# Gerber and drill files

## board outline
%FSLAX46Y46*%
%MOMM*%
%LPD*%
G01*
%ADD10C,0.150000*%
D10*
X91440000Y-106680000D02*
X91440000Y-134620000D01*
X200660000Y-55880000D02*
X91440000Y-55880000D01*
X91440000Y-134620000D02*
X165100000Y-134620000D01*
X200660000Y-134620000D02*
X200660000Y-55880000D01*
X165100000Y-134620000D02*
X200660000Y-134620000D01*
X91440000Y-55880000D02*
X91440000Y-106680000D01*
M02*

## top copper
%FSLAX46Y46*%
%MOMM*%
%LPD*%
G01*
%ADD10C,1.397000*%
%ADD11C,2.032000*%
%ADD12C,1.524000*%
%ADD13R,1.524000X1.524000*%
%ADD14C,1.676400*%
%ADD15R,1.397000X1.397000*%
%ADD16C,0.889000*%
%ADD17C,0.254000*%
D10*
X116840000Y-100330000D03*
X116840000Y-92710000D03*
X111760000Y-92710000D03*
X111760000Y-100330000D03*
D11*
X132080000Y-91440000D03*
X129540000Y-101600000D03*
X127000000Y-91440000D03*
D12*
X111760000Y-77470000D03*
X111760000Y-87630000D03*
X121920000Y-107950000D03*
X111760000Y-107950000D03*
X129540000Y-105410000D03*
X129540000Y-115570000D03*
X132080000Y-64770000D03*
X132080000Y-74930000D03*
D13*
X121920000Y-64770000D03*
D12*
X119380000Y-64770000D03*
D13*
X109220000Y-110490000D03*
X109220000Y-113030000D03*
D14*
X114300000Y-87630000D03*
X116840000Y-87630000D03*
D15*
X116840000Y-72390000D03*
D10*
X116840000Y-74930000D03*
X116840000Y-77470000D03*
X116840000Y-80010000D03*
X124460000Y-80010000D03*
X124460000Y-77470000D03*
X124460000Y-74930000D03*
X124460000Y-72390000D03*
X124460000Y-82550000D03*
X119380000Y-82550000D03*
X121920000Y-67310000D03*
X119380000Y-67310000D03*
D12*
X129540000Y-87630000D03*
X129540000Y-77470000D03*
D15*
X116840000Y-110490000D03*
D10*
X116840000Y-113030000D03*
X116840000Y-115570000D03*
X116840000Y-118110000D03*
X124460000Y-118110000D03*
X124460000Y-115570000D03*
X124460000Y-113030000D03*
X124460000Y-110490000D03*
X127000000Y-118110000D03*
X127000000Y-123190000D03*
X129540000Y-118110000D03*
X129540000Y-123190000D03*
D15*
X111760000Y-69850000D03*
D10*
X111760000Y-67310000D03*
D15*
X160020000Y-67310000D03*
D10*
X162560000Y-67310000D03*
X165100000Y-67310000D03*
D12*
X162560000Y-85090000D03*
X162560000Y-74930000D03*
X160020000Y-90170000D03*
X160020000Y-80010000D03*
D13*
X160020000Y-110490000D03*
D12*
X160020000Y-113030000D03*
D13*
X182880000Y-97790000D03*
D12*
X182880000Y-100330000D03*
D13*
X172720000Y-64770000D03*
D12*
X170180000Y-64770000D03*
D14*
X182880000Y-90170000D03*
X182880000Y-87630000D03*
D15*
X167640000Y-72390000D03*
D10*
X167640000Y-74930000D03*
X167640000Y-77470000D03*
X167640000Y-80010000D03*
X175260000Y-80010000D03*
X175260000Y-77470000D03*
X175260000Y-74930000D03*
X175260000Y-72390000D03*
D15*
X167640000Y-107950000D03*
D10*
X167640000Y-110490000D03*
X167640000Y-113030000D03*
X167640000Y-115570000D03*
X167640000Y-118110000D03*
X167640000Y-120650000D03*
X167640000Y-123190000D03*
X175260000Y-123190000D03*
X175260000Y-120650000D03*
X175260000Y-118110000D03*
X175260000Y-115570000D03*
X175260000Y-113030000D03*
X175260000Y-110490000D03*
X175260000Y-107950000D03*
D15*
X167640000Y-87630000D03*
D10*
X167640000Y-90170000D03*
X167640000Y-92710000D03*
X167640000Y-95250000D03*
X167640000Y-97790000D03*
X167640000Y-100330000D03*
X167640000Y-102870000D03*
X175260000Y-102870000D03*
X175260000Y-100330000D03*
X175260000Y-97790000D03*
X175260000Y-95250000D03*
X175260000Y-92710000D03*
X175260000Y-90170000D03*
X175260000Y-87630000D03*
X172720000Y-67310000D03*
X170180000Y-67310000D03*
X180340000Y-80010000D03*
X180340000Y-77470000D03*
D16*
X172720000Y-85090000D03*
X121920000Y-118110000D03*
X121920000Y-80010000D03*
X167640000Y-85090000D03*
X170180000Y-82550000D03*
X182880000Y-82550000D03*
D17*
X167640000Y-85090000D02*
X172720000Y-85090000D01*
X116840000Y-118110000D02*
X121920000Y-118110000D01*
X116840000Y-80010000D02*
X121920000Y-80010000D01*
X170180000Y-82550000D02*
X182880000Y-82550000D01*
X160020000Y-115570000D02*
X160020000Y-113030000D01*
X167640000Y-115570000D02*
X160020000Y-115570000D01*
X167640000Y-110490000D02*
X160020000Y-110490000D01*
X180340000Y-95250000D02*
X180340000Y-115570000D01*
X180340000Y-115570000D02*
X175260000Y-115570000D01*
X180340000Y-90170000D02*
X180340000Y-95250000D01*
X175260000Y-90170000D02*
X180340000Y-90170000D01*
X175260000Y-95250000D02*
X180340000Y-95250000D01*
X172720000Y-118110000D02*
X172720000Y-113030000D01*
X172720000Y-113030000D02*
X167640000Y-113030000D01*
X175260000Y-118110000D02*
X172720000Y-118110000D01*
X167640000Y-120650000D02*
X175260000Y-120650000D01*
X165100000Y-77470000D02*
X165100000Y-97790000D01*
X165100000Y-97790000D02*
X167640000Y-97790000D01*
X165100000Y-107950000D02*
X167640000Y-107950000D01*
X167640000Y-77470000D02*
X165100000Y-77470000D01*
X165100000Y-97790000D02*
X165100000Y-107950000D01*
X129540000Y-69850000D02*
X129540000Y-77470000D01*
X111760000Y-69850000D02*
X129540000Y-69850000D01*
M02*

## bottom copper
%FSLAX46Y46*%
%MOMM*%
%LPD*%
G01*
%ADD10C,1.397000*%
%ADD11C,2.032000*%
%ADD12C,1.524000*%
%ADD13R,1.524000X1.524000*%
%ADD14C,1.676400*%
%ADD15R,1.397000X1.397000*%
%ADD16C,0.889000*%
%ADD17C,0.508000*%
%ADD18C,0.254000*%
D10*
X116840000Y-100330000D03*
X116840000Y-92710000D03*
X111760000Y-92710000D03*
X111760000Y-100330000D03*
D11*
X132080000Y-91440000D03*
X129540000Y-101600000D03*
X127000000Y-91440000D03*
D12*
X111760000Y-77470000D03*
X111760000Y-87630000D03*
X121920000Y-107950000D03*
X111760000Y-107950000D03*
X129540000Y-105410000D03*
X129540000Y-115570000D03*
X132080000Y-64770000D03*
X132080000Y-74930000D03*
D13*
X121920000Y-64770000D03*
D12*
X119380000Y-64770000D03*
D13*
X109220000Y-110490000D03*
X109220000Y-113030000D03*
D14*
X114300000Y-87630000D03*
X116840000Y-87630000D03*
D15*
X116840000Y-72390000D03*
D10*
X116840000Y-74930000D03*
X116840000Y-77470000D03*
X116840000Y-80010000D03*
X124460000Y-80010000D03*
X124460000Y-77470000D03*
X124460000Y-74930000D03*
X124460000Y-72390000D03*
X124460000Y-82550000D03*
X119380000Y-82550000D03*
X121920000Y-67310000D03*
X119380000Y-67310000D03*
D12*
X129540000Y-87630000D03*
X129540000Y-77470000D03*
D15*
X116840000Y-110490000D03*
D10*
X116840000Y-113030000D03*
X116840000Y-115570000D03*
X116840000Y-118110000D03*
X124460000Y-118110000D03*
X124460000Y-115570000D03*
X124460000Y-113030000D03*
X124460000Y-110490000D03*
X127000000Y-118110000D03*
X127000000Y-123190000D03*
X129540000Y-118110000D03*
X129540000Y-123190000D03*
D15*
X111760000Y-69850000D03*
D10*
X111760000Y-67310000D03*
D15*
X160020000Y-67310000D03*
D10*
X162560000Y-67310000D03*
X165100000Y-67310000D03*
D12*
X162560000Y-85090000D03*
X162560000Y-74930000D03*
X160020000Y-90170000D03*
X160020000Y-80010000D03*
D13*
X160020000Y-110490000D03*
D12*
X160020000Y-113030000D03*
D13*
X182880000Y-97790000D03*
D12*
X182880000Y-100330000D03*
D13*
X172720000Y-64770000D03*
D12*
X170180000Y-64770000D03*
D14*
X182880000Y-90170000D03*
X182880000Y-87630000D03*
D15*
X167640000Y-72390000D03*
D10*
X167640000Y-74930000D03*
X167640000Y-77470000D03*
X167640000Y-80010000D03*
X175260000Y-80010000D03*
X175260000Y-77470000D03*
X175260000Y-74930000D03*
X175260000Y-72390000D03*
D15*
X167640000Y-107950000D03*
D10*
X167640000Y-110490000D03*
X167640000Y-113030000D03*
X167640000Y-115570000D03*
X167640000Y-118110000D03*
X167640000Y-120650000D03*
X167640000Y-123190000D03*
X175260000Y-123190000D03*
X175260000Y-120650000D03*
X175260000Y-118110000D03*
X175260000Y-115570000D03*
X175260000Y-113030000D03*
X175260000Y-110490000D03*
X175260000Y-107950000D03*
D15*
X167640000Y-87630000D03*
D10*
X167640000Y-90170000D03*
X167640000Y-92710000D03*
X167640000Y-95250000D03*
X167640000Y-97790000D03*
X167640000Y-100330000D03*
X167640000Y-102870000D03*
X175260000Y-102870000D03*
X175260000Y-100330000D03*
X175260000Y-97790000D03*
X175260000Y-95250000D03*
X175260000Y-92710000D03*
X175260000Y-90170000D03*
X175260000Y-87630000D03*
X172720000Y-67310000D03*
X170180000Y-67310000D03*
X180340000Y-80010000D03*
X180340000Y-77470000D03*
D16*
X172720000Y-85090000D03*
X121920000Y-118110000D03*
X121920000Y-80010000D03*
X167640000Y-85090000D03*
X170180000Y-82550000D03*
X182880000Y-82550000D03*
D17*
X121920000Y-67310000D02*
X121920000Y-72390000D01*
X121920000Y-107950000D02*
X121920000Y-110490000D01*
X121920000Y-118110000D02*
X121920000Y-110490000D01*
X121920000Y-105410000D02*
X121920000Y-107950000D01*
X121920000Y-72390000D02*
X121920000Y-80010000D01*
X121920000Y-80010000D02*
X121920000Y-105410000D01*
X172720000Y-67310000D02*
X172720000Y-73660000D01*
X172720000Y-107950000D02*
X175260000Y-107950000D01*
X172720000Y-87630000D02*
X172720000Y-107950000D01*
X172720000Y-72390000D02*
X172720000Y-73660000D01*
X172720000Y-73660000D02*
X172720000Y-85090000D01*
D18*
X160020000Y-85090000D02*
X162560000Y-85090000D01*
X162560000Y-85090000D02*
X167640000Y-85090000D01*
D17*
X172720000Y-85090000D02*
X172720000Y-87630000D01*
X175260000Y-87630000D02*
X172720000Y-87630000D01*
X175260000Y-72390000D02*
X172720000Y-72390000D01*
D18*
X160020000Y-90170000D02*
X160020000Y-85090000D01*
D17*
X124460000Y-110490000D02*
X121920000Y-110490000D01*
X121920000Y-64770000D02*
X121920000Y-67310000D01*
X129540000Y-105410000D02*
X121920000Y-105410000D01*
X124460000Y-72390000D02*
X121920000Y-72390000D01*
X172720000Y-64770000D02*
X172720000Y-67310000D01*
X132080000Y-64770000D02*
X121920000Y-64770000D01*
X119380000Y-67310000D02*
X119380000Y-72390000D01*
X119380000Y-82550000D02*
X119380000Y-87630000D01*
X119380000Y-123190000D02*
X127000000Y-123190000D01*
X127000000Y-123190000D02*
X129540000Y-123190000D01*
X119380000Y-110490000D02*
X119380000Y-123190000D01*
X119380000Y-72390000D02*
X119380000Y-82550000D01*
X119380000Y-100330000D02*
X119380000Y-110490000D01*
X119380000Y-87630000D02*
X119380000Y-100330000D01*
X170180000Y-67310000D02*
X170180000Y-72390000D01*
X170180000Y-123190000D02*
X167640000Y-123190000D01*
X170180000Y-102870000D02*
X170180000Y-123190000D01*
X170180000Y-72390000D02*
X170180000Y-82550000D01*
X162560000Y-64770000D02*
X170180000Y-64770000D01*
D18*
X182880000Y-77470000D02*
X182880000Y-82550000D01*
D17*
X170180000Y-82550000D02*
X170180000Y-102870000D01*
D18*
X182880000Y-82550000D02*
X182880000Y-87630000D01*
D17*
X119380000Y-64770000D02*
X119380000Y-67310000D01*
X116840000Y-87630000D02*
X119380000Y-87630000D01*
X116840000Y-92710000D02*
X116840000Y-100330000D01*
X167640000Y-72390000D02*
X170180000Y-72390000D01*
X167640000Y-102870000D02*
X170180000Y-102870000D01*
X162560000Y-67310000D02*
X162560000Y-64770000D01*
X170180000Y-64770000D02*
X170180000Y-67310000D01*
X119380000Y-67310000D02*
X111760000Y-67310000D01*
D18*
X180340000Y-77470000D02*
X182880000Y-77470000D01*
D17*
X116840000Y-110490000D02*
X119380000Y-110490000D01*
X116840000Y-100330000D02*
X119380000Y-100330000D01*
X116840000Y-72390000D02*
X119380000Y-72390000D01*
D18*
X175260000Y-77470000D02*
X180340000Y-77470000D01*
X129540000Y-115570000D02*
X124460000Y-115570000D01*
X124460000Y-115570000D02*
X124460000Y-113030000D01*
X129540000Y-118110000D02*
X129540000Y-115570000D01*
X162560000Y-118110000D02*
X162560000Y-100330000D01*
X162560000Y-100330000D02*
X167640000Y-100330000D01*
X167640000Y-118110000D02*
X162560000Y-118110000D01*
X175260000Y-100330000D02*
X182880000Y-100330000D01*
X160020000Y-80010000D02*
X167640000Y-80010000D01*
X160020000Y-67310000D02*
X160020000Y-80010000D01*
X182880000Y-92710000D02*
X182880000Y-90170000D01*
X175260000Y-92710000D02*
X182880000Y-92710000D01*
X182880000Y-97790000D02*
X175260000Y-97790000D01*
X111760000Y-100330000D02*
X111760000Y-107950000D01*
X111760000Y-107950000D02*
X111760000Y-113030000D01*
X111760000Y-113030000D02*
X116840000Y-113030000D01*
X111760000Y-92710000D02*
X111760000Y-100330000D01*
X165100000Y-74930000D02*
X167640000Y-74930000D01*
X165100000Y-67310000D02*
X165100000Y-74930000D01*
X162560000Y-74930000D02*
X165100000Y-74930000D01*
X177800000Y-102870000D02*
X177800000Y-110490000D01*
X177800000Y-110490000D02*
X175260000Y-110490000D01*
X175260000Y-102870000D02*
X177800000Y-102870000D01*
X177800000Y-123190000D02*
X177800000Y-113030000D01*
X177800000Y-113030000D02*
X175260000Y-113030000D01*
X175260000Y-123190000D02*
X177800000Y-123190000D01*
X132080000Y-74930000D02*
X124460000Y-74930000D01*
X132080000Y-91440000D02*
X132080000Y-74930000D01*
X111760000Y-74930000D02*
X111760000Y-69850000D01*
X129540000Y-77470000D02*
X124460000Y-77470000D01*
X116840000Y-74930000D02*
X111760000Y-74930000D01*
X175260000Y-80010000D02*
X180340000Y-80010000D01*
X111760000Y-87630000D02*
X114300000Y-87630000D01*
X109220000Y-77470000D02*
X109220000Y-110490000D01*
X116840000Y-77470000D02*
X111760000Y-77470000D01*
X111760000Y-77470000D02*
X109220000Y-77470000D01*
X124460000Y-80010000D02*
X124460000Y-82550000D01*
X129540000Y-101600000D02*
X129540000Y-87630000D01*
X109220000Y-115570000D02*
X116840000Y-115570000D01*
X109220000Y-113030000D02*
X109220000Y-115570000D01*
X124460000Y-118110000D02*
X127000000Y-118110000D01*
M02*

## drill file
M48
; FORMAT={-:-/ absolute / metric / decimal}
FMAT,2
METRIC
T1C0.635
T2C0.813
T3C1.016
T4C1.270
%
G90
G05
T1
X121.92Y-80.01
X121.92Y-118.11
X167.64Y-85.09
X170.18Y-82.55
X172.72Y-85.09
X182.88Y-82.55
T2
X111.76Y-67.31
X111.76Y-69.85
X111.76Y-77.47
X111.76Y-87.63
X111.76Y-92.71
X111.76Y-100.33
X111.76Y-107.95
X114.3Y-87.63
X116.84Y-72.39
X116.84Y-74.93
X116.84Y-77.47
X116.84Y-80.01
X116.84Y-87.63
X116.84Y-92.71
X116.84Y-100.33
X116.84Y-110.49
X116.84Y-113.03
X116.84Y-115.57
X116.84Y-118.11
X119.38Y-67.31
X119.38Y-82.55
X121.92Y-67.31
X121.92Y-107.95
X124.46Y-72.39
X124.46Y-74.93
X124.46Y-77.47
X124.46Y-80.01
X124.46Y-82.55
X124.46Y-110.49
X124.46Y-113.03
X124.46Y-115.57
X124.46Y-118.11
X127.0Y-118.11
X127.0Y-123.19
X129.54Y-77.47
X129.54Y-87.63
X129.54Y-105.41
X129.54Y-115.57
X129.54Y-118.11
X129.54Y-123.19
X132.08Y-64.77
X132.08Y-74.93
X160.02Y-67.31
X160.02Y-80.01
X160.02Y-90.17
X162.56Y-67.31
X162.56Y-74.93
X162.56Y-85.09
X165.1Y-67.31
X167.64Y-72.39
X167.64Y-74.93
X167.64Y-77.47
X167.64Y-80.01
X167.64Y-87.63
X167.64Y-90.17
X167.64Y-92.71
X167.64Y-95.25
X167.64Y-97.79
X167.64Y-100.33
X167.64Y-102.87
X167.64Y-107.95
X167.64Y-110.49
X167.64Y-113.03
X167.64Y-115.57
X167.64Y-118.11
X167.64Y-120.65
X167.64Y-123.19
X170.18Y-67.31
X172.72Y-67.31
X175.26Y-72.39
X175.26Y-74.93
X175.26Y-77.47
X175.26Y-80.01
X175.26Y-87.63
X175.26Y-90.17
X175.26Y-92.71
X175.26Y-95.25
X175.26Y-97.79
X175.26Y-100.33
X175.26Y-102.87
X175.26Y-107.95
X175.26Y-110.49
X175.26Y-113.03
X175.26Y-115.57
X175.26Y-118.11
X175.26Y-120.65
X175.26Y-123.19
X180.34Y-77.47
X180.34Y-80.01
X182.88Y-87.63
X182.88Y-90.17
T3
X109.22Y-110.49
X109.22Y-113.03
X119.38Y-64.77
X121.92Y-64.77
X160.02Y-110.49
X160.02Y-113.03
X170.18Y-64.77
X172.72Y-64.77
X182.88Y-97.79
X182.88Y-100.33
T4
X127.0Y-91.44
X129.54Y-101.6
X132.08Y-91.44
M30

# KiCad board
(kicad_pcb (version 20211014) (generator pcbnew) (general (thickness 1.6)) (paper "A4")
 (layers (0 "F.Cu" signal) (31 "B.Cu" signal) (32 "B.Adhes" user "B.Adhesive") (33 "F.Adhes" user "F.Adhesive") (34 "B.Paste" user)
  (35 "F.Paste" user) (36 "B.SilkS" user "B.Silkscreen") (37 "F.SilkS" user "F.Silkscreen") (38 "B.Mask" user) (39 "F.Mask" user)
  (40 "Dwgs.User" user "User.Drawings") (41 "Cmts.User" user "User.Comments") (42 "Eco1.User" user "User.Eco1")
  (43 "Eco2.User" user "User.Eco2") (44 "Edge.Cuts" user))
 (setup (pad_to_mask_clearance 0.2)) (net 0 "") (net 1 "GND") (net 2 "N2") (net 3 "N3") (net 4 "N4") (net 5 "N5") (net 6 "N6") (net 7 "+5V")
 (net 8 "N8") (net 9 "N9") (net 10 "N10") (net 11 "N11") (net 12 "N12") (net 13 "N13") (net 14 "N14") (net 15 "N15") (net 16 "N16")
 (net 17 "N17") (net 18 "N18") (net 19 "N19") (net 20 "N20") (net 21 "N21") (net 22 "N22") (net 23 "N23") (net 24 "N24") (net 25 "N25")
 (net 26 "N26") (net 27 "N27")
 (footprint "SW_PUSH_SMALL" (layer "F.Cu") (at 114.3 96.52 -90)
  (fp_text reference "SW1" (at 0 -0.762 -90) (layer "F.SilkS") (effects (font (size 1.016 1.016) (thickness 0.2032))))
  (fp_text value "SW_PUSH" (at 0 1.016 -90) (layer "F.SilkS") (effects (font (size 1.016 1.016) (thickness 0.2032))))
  (pad "1" thru_hole circle locked (at 3.81 -2.54 270) (size 1.397 1.397) (drill 0.8128) (layers *.Cu *.Mask "F.SilkS") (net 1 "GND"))
  (pad "1" thru_hole circle locked (at -3.81 -2.54 270) (size 1.397 1.397) (drill 0.8128) (layers *.Cu *.Mask "F.SilkS") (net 1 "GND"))
  (pad "2" thru_hole circle locked (at -3.81 2.54 270) (size 1.397 1.397) (drill 0.8128) (layers *.Cu *.Mask "F.SilkS") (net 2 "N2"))
  (pad "2" thru_hole circle locked (at 3.81 2.54 270) (size 1.397 1.397) (drill 0.8128) (layers *.Cu *.Mask "F.SilkS") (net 2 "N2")))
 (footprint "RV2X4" (layer "F.Cu") (at 129.54 96.52 -90)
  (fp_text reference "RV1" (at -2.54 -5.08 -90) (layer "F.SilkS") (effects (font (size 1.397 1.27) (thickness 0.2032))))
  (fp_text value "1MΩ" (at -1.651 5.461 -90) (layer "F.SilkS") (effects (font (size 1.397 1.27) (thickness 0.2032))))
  (pad "1" thru_hole circle locked (at -5.08 -2.54 270) (size 2.032 2.032) (drill 1.27) (layers *.Cu *.Mask "F.SilkS") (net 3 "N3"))
  (pad "2" thru_hole circle locked (at 5.08 0 270) (size 2.032 2.032) (drill 1.27) (layers *.Cu *.Mask "F.SilkS") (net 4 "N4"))
  (pad "3" thru_hole circle locked (at -5.08 2.54 270) (size 2.032 2.032) (drill 1.27) (layers *.Cu *.Mask "F.SilkS")))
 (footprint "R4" (layer "F.Cu") (at 111.76 82.55 -90) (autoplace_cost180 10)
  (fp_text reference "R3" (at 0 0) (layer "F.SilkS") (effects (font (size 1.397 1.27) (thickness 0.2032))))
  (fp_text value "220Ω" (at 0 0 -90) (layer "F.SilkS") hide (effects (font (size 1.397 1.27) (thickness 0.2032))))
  (pad "1" thru_hole circle locked (at -5.08 0 270) (size 1.524 1.524) (drill 0.8128) (layers *.Cu *.Mask "F.SilkS") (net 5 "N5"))
  (pad "2" thru_hole circle locked (at 5.08 0 270) (size 1.524 1.524) (drill 0.8128) (layers *.Cu *.Mask "F.SilkS") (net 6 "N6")))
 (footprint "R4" (layer "F.Cu") (at 116.84 107.95 180) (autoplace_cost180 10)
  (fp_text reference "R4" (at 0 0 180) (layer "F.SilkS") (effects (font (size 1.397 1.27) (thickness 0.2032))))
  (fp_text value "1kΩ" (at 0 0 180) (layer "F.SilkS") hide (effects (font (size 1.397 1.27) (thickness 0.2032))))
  (pad "1" thru_hole circle locked (at -5.08 0 180) (size 1.524 1.524) (drill 0.8128) (layers *.Cu *.Mask "F.SilkS") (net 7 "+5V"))
  (pad "2" thru_hole circle locked (at 5.08 0 180) (size 1.524 1.524) (drill 0.8128) (layers *.Cu *.Mask "F.SilkS") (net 2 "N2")))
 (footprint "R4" (layer "F.Cu") (at 129.54 110.49 -90) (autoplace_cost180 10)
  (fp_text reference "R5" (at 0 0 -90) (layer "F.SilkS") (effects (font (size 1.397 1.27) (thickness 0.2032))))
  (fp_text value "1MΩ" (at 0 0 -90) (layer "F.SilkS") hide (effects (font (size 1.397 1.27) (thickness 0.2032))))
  (pad "1" thru_hole circle locked (at -5.08 0 270) (size 1.524 1.524) (drill 0.8128) (layers *.Cu *.Mask "F.SilkS") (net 7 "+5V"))
  (pad "2" thru_hole circle locked (at 5.08 0 270) (size 1.524 1.524) (drill 0.8128) (layers *.Cu *.Mask "F.SilkS") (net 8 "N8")))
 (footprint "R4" (layer "F.Cu") (at 132.08 69.85 -90) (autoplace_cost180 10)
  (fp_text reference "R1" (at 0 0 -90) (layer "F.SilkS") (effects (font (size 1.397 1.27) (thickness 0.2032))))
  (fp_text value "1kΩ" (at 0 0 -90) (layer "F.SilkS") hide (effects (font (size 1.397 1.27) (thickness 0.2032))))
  (pad "1" thru_hole circle locked (at -5.08 0 270) (size 1.524 1.524) (drill 0.8128) (layers *.Cu *.Mask "F.SilkS") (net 7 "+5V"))
  (pad "2" thru_hole circle locked (at 5.08 0 270) (size 1.524 1.524) (drill 0.8128) (layers *.Cu *.Mask "F.SilkS") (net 3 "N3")))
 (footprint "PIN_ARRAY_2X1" (layer "F.Cu") (at 120.65 64.77 180)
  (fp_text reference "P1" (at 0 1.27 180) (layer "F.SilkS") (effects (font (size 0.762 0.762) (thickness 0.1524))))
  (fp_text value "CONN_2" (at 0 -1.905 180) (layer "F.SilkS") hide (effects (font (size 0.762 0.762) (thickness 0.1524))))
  (pad "1" thru_hole rect locked (at -1.27 0 180) (size 1.524 1.524) (drill 1.016) (layers *.Cu *.Mask "F.SilkS") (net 7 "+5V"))
  (pad "2" thru_hole circle locked (at 1.27 0 180) (size 1.524 1.524) (drill 1.016) (layers *.Cu *.Mask "F.SilkS") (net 1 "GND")))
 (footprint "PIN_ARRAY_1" (layer "F.Cu") (at 109.22 110.49)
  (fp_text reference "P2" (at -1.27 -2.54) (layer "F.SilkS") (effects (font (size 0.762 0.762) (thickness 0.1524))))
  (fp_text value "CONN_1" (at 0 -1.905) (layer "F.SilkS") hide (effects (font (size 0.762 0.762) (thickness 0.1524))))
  (pad "1" thru_hole rect locked (at 0 0) (size 1.524 1.524) (drill 1.016) (layers *.Cu *.Mask "F.SilkS") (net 5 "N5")))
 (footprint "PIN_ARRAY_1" (layer "F.Cu") (at 109.22 113.03)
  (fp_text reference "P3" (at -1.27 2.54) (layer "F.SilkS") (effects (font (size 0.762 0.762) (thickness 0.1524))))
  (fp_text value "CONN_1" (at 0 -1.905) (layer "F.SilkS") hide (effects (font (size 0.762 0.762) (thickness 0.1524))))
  (pad "1" thru_hole rect locked (at 0 0) (size 1.524 1.524) (drill 1.016) (layers *.Cu *.Mask "F.SilkS") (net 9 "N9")))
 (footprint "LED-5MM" (layer "F.Cu") (at 115.57 87.63)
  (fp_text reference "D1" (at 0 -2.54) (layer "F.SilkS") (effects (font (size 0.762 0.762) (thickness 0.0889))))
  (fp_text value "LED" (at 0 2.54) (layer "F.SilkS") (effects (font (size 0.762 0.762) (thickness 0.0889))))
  (pad "1" thru_hole circle locked (at -1.27 0) (size 1.6764 1.6764) (drill 0.8128) (layers *.Cu *.Mask "F.SilkS") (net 6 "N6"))
  (pad "2" thru_hole circle locked (at 1.27 0) (size 1.6764 1.6764) (drill 0.8128) (layers *.Cu *.Mask "F.SilkS") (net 1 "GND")))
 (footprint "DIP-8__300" (layer "F.Cu") (at 120.65 76.2 -90)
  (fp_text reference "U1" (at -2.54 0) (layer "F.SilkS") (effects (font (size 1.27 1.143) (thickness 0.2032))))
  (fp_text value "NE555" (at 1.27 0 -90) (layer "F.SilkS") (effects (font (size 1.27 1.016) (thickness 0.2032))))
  (pad "1" thru_hole rect locked (at -3.81 3.81 270) (size 1.397 1.397) (drill 0.8128) (layers *.Cu *.Mask "F.SilkS") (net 1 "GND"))
  (pad "2" thru_hole circle locked (at -1.27 3.81 270) (size 1.397 1.397) (drill 0.8128) (layers *.Cu *.Mask "F.SilkS") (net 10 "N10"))
  (pad "3" thru_hole circle locked (at 1.27 3.81 270) (size 1.397 1.397) (drill 0.8128) (layers *.Cu *.Mask "F.SilkS") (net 5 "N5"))
  (pad "4" thru_hole circle locked (at 3.81 3.81 270) (size 1.397 1.397) (drill 0.8128) (layers *.Cu *.Mask "F.SilkS") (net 7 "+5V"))
  (pad "5" thru_hole circle locked (at 3.81 -3.81 270) (size 1.397 1.397) (drill 0.8128) (layers *.Cu *.Mask "F.SilkS") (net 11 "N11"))
  (pad "6" thru_hole circle locked (at 1.27 -3.81 270) (size 1.397 1.397) (drill 0.8128) (layers *.Cu *.Mask "F.SilkS") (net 10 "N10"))
  (pad "7" thru_hole circle locked (at -1.27 -3.81 270) (size 1.397 1.397) (drill 0.8128) (layers *.Cu *.Mask "F.SilkS") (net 3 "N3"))
  (pad "8" thru_hole circle locked (at -3.81 -3.81 270) (size 1.397 1.397) (drill 0.8128) (layers *.Cu *.Mask "F.SilkS") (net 7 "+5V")))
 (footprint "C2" (layer "F.Cu") (at 121.92 82.55 180)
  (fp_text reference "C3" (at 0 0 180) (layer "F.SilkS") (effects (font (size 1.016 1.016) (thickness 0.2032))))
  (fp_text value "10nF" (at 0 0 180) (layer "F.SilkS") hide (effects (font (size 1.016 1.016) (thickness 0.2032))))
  (pad "1" thru_hole circle locked (at -2.54 0 180) (size 1.397 1.397) (drill 0.8128) (layers *.Cu *.Mask "F.SilkS") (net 11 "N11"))
  (pad "2" thru_hole circle locked (at 2.54 0 180) (size 1.397 1.397) (drill 0.8128) (layers *.Cu *.Mask "F.SilkS") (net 1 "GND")))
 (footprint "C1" (layer "F.Cu") (at 120.65 67.31 180)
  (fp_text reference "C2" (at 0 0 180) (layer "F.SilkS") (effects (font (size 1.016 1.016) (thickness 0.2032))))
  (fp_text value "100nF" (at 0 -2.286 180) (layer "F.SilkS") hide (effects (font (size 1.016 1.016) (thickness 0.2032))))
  (pad "1" thru_hole circle locked (at -1.27 0 180) (size 1.397 1.397) (drill 0.8128) (layers *.Cu *.Mask "F.SilkS") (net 7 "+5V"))
  (pad "2" thru_hole circle locked (at 1.27 0 180) (size 1.397 1.397) (drill 0.8128) (layers *.Cu *.Mask "F.SilkS") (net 1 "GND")))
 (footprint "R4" (layer "F.Cu") (at 129.54 82.55 90) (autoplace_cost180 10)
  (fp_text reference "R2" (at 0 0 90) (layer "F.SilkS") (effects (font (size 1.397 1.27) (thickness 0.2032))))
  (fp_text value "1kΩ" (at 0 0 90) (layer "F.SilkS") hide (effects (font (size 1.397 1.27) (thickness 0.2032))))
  (pad "1" thru_hole circle locked (at -5.08 0 90) (size 1.524 1.524) (drill 0.8128) (layers *.Cu *.Mask "F.SilkS") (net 4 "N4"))
  (pad "2" thru_hole circle locked (at 5.08 0 90) (size 1.524 1.524) (drill 0.8128) (layers *.Cu *.Mask "F.SilkS") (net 10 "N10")))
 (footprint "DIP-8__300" (layer "F.Cu") (at 120.65 114.3 -90)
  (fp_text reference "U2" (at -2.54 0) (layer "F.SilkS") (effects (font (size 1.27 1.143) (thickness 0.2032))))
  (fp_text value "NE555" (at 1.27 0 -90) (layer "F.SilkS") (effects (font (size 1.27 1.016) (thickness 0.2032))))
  (pad "1" thru_hole rect locked (at -3.81 3.81 270) (size 1.397 1.397) (drill 0.8128) (layers *.Cu *.Mask "F.SilkS") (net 1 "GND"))
  (pad "2" thru_hole circle locked (at -1.27 3.81 270) (size 1.397 1.397) (drill 0.8128) (layers *.Cu *.Mask "F.SilkS") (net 2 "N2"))
  (pad "3" thru_hole circle locked (at 1.27 3.81 270) (size 1.397 1.397) (drill 0.8128) (layers *.Cu *.Mask "F.SilkS") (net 9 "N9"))
  (pad "4" thru_hole circle locked (at 3.81 3.81 270) (size 1.397 1.397) (drill 0.8128) (layers *.Cu *.Mask "F.SilkS") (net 7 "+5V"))
  (pad "5" thru_hole circle locked (at 3.81 -3.81 270) (size 1.397 1.397) (drill 0.8128) (layers *.Cu *.Mask "F.SilkS") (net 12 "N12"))
  (pad "6" thru_hole circle locked (at 1.27 -3.81 270) (size 1.397 1.397) (drill 0.8128) (layers *.Cu *.Mask "F.SilkS") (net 8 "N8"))
  (pad "7" thru_hole circle locked (at -1.27 -3.81 270) (size 1.397 1.397) (drill 0.8128) (layers *.Cu *.Mask "F.SilkS") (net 8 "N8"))
  (pad "8" thru_hole circle locked (at -3.81 -3.81 270) (size 1.397 1.397) (drill 0.8128) (layers *.Cu *.Mask "F.SilkS") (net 7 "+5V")))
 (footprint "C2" (layer "F.Cu") (at 127 120.65 -90)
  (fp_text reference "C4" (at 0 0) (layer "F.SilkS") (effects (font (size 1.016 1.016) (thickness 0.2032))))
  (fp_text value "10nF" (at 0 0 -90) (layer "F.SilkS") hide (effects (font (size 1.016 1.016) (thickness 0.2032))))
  (pad "1" thru_hole circle locked (at -2.54 0 270) (size 1.397 1.397) (drill 0.8128) (layers *.Cu *.Mask "F.SilkS") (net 12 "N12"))
  (pad "2" thru_hole circle locked (at 2.54 0 270) (size 1.397 1.397) (drill 0.8128) (layers *.Cu *.Mask "F.SilkS") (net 1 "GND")))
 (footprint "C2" (layer "F.Cu") (at 129.54 120.65 -90)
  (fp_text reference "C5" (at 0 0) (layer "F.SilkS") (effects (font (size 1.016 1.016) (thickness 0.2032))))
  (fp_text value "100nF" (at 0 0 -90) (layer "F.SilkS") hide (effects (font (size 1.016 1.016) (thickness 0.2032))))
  (pad "1" thru_hole circle locked (at -2.54 0 270) (size 1.397 1.397) (drill 0.8128) (layers *.Cu *.Mask "F.SilkS") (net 8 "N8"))
  (pad "2" thru_hole circle locked (at 2.54 0 270) (size 1.397 1.397) (drill 0.8128) (layers *.Cu *.Mask "F.SilkS") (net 1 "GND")))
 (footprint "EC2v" (layer "F.Cu") (at 111.76 68.58 90)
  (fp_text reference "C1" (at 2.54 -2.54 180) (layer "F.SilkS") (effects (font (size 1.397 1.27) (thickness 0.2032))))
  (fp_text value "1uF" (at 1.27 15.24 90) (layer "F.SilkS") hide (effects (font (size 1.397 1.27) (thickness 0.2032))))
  (pad "1" thru_hole rect locked (at -1.27 0 90) (size 1.397 1.397) (drill 0.8128) (layers *.Cu *.Mask "F.SilkS") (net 10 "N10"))
  (pad "2" thru_hole circle locked (at 1.27 0 90) (size 1.397 1.397) (drill 0.8128) (layers *.Cu *.Mask "F.SilkS") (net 1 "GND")))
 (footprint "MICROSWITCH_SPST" (layer "F.Cu") (at 162.56 67.31)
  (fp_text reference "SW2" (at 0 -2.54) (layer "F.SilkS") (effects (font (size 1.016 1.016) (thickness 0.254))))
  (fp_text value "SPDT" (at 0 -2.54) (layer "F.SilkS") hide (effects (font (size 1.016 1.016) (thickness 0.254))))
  (pad "1" thru_hole rect locked (at -2.54 0) (size 1.397 1.397) (drill 0.8128) (layers *.Cu *.Mask "F.SilkS") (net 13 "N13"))
  (pad "2" thru_hole circle locked (at 0 0) (size 1.397 1.397) (drill 0.8128) (layers *.Cu *.Mask "F.SilkS") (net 1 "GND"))
  (pad "3" thru_hole circle locked (at 2.54 0) (size 1.397 1.397) (drill 0.8128) (layers *.Cu *.Mask "F.SilkS") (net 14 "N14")))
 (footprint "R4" (layer "F.Cu") (at 162.56 80.01 90) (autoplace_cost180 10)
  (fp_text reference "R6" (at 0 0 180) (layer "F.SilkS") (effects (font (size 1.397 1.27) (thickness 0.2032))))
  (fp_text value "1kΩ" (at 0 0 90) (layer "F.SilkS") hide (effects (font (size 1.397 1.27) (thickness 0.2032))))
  (pad "1" thru_hole circle locked (at -5.08 0 90) (size 1.524 1.524) (drill 0.8128) (layers *.Cu *.Mask "F.SilkS") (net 7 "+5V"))
  (pad "2" thru_hole circle locked (at 5.08 0 90) (size 1.524 1.524) (drill 0.8128) (layers *.Cu *.Mask "F.SilkS") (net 14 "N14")))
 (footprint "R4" (layer "F.Cu") (at 160.02 85.09 90) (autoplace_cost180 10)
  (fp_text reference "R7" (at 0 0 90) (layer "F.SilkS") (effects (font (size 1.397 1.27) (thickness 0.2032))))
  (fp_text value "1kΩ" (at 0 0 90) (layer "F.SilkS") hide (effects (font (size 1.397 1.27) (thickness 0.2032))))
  (pad "1" thru_hole circle locked (at -5.08 0 90) (size 1.524 1.524) (drill 0.8128) (layers *.Cu *.Mask "F.SilkS") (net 7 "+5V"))
  (pad "2" thru_hole circle locked (at 5.08 0 90) (size 1.524 1.524) (drill 0.8128) (layers *.Cu *.Mask "F.SilkS") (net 13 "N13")))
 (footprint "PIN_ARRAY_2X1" (layer "F.Cu") (at 160.02 111.76 -90)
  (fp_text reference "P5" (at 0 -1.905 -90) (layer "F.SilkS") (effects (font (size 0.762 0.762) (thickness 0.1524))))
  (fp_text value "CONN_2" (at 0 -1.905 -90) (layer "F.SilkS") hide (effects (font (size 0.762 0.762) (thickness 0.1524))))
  (pad "1" thru_hole rect locked (at -1.27 0 270) (size 1.524 1.524) (drill 1.016) (layers *.Cu *.Mask "F.SilkS") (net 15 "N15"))
  (pad "2" thru_hole circle locked (at 1.27 0 270) (size 1.524 1.524) (drill 1.016) (layers *.Cu *.Mask "F.SilkS") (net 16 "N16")))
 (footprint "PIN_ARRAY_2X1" (layer "F.Cu") (at 182.88 99.06 -90)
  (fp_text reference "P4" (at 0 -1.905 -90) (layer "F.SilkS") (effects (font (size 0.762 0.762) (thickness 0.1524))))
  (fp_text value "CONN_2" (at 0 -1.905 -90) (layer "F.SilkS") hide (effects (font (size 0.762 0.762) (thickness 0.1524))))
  (pad "1" thru_hole rect locked (at -1.27 0 270) (size 1.524 1.524) (drill 1.016) (layers *.Cu *.Mask "F.SilkS") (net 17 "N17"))
  (pad "2" thru_hole circle locked (at 1.27 0 270) (size 1.524 1.524) (drill 1.016) (layers *.Cu *.Mask "F.SilkS") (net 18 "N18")))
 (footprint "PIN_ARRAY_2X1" (layer "F.Cu") (at 171.45 64.77 180)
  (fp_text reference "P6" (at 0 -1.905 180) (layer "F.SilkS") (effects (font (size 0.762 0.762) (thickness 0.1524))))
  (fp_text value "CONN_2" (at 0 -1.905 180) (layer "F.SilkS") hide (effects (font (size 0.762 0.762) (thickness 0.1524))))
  (pad "1" thru_hole rect locked (at -1.27 0 180) (size 1.524 1.524) (drill 1.016) (layers *.Cu *.Mask "F.SilkS") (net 7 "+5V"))
  (pad "2" thru_hole circle locked (at 1.27 0 180) (size 1.524 1.524) (drill 1.016) (layers *.Cu *.Mask "F.SilkS") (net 1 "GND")))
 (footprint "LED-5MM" (layer "F.Cu") (at 182.88 88.9 90)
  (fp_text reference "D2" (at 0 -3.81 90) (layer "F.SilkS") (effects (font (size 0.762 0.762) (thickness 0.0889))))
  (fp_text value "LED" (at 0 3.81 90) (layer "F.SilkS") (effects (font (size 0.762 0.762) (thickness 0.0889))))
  (pad "1" thru_hole circle locked (at -1.27 0 90) (size 1.6764 1.6764) (drill 0.8128) (layers *.Cu *.Mask "F.SilkS") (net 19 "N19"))
  (pad "2" thru_hole circle locked (at 1.27 0 90) (size 1.6764 1.6764) (drill 0.8128) (layers *.Cu *.Mask "F.SilkS") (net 1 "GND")))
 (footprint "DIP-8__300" (layer "F.Cu") (at 171.45 76.2 -90)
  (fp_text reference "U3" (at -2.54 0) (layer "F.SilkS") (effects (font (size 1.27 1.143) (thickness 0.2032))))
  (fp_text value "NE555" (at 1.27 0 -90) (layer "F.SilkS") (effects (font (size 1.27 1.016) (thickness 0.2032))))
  (pad "1" thru_hole rect locked (at -3.81 3.81 270) (size 1.397 1.397) (drill 0.8128) (layers *.Cu *.Mask "F.SilkS") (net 1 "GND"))
  (pad "2" thru_hole circle locked (at -1.27 3.81 270) (size 1.397 1.397) (drill 0.8128) (layers *.Cu *.Mask "F.SilkS") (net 14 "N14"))
  (pad "3" thru_hole circle locked (at 1.27 3.81 270) (size 1.397 1.397) (drill 0.8128) (layers *.Cu *.Mask "F.SilkS") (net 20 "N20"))
  (pad "4" thru_hole circle locked (at 3.81 3.81 270) (size 1.397 1.397) (drill 0.8128) (layers *.Cu *.Mask "F.SilkS") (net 13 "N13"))
  (pad "5" thru_hole circle locked (at 3.81 -3.81 270) (size 1.397 1.397) (drill 0.8128) (layers *.Cu *.Mask "F.SilkS") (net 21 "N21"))
  (pad "6" thru_hole circle locked (at 1.27 -3.81 270) (size 1.397 1.397) (drill 0.8128) (layers *.Cu *.Mask "F.SilkS") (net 1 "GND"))
  (pad "7" thru_hole circle locked (at -1.27 -3.81 270) (size 1.397 1.397) (drill 0.8128) (layers *.Cu *.Mask "F.SilkS"))
  (pad "8" thru_hole circle locked (at -3.81 -3.81 270) (size 1.397 1.397) (drill 0.8128) (layers *.Cu *.Mask "F.SilkS") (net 7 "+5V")))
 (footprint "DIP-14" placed (layer "F.Cu") (at 171.45 115.57 -90)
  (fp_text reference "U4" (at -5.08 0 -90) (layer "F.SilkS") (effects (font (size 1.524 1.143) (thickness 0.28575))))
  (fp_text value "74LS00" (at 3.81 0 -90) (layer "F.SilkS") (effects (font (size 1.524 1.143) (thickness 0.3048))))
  (pad "1" thru_hole rect locked (at -7.62 3.81 270) (size 1.397 1.397) (drill 0.8128) (layers *.Cu *.Mask "F.SilkS") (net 20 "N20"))
  (pad "2" thru_hole circle locked (at -5.08 3.81 270) (size 1.397 1.397) (drill 0.8128) (layers *.Cu *.Mask "F.SilkS") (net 15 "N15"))
  (pad "3" thru_hole circle locked (at -2.54 3.81 270) (size 1.397 1.397) (drill 0.8128) (layers *.Cu *.Mask "F.SilkS") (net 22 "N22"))
  (pad "4" thru_hole circle locked (at 0 3.81 270) (size 1.397 1.397) (drill 0.8128) (layers *.Cu *.Mask "F.SilkS") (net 16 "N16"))
  (pad "5" thru_hole circle locked (at 2.54 3.81 270) (size 1.397 1.397) (drill 0.8128) (layers *.Cu *.Mask "F.SilkS") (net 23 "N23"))
  (pad "6" thru_hole circle locked (at 5.08 3.81 270) (size 1.397 1.397) (drill 0.8128) (layers *.Cu *.Mask "F.SilkS") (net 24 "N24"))
  (pad "7" thru_hole circle locked (at 7.62 3.81 270) (size 1.397 1.397) (drill 0.8128) (layers *.Cu *.Mask "F.SilkS") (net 1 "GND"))
  (pad "8" thru_hole circle locked (at 7.62 -3.81 270) (size 1.397 1.397) (drill 0.8128) (layers *.Cu *.Mask "F.SilkS") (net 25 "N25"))
  (pad "9" thru_hole circle locked (at 5.08 -3.81 270) (size 1.397 1.397) (drill 0.8128) (layers *.Cu *.Mask "F.SilkS") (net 24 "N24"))
  (pad "10" thru_hole circle locked (at 2.54 -3.81 270) (size 1.397 1.397) (drill 0.8128) (layers *.Cu *.Mask "F.SilkS") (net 22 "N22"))
  (pad "11" thru_hole circle locked (at 0 -3.81 270) (size 1.397 1.397) (drill 0.8128) (layers *.Cu *.Mask "F.SilkS") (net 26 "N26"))
  (pad "12" thru_hole circle locked (at -2.54 -3.81 270) (size 1.397 1.397) (drill 0.8128) (layers *.Cu *.Mask "F.SilkS") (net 25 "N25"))
  (pad "13" thru_hole circle locked (at -5.08 -3.81 270) (size 1.397 1.397) (drill 0.8128) (layers *.Cu *.Mask "F.SilkS") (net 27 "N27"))
  (pad "14" thru_hole circle locked (at -7.62 -3.81 270) (size 1.397 1.397) (drill 0.8128) (layers *.Cu *.Mask "F.SilkS") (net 7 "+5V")))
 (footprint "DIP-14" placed (layer "F.Cu") (at 171.45 95.25 -90)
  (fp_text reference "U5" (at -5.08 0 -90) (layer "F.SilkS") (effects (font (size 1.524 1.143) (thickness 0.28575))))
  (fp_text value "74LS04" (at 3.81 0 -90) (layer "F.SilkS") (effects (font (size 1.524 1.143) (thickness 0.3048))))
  (pad "1" thru_hole rect locked (at -7.62 3.81 270) (size 1.397 1.397) (drill 0.8128) (layers *.Cu *.Mask "F.SilkS"))
  (pad "2" thru_hole circle locked (at -5.08 3.81 270) (size 1.397 1.397) (drill 0.8128) (layers *.Cu *.Mask "F.SilkS"))
  (pad "3" thru_hole circle locked (at -2.54 3.81 270) (size 1.397 1.397) (drill 0.8128) (layers *.Cu *.Mask "F.SilkS"))
  (pad "4" thru_hole circle locked (at 0 3.81 270) (size 1.397 1.397) (drill 0.8128) (layers *.Cu *.Mask "F.SilkS"))
  (pad "5" thru_hole circle locked (at 2.54 3.81 270) (size 1.397 1.397) (drill 0.8128) (layers *.Cu *.Mask "F.SilkS") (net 20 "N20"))
  (pad "6" thru_hole circle locked (at 5.08 3.81 270) (size 1.397 1.397) (drill 0.8128) (layers *.Cu *.Mask "F.SilkS") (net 23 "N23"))
  (pad "7" thru_hole circle locked (at 7.62 3.81 270) (size 1.397 1.397) (drill 0.8128) (layers *.Cu *.Mask "F.SilkS") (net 1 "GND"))
  (pad "8" thru_hole circle locked (at 7.62 -3.81 270) (size 1.397 1.397) (drill 0.8128) (layers *.Cu *.Mask "F.SilkS") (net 27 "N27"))
  (pad "9" thru_hole circle locked (at 5.08 -3.81 270) (size 1.397 1.397) (drill 0.8128) (layers *.Cu *.Mask "F.SilkS") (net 18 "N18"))
  (pad "10" thru_hole circle locked (at 2.54 -3.81 270) (size 1.397 1.397) (drill 0.8128) (layers *.Cu *.Mask "F.SilkS") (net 17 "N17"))
  (pad "11" thru_hole circle locked (at 0 -3.81 270) (size 1.397 1.397) (drill 0.8128) (layers *.Cu *.Mask "F.SilkS") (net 26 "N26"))
  (pad "12" thru_hole circle locked (at -2.54 -3.81 270) (size 1.397 1.397) (drill 0.8128) (layers *.Cu *.Mask "F.SilkS") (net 19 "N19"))
  (pad "13" thru_hole circle locked (at -5.08 -3.81 270) (size 1.397 1.397) (drill 0.8128) (layers *.Cu *.Mask "F.SilkS") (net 26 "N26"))
  (pad "14" thru_hole circle locked (at -7.62 -3.81 270) (size 1.397 1.397) (drill 0.8128) (layers *.Cu *.Mask "F.SilkS") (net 7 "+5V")))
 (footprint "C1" (layer "F.Cu") (at 171.45 67.31 180)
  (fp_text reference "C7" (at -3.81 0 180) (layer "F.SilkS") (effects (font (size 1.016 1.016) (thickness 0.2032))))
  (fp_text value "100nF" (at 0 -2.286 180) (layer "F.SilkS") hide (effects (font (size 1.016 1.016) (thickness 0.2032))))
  (pad "1" thru_hole circle locked (at -1.27 0 180) (size 1.397 1.397) (drill 0.8128) (layers *.Cu *.Mask "F.SilkS") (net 7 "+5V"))
  (pad "2" thru_hole circle locked (at 1.27 0 180) (size 1.397 1.397) (drill 0.8128) (layers *.Cu *.Mask "F.SilkS") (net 1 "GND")))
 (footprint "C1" (layer "F.Cu") (at 180.34 78.74 90)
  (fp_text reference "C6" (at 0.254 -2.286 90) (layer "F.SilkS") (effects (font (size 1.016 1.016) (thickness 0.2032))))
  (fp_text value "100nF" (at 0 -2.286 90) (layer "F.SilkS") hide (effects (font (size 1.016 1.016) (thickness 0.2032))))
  (pad "1" thru_hole circle locked (at -1.27 0 90) (size 1.397 1.397) (drill 0.8128) (layers *.Cu *.Mask "F.SilkS") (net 21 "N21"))
  (pad "2" thru_hole circle locked (at 1.27 0 90) (size 1.397 1.397) (drill 0.8128) (layers *.Cu *.Mask "F.SilkS") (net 1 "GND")))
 (gr_line (start 91.44 106.68) (end 91.44 134.62) (layer "Edge.Cuts") (width 0.15))
 (gr_line (start 200.66 55.88) (end 91.44 55.88) (layer "Edge.Cuts") (width 0.15))
 (gr_line (start 91.44 134.62) (end 165.1 134.62) (layer "Edge.Cuts") (width 0.15))
 (gr_line (start 200.66 134.62) (end 200.66 55.88) (layer "Edge.Cuts") (width 0.15))
 (gr_line (start 165.1 134.62) (end 200.66 134.62) (layer "Edge.Cuts") (width 0.15))
 (gr_line (start 91.44 55.88) (end 91.44 106.68) (layer "Edge.Cuts") (width 0.15))
 (segment (start 167.64 85.09) (end 172.72 85.09) (width 0.254) (layer "F.Cu") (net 7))
 (segment (start 116.84 118.11) (end 121.92 118.11) (width 0.254) (layer "F.Cu") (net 7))
 (segment (start 116.84 80.01) (end 121.92 80.01) (width 0.254) (layer "F.Cu") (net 7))
 (via (at 172.72 85.09) (size 0.889) (drill 0.635) (layers "F.Cu" "B.Cu") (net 7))
 (via (at 121.92 118.11) (size 0.889) (drill 0.635) (layers "F.Cu" "B.Cu") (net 7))
 (via (at 121.92 80.01) (size 0.889) (drill 0.635) (layers "F.Cu" "B.Cu") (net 7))
 (via (at 167.64 85.09) (size 0.889) (drill 0.635) (layers "F.Cu" "B.Cu") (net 7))
 (segment (start 121.92 67.31) (end 121.92 72.39) (width 0.508) (layer "B.Cu") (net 7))
 (segment (start 121.92 107.95) (end 121.92 110.49) (width 0.508) (layer "B.Cu") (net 7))
 (segment (start 121.92 118.11) (end 121.92 110.49) (width 0.508) (layer "B.Cu") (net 7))
 (segment (start 121.92 105.41) (end 121.92 107.95) (width 0.508) (layer "B.Cu") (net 7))
 (segment (start 121.92 72.39) (end 121.92 80.01) (width 0.508) (layer "B.Cu") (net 7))
 (segment (start 121.92 80.01) (end 121.92 105.41) (width 0.508) (layer "B.Cu") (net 7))
 (segment (start 172.72 67.31) (end 172.72 73.66) (width 0.508) (layer "B.Cu") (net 7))
 (segment (start 172.72 107.95) (end 175.26 107.95) (width 0.508) (layer "B.Cu") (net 7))
 (segment (start 172.72 87.63) (end 172.72 107.95) (width 0.508) (layer "B.Cu") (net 7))
 (segment (start 172.72 72.39) (end 172.72 73.66) (width 0.508) (layer "B.Cu") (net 7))
 (segment (start 172.72 73.66) (end 172.72 85.09) (width 0.508) (layer "B.Cu") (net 7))
 (segment (start 160.02 85.09) (end 162.56 85.09) (width 0.254) (layer "B.Cu") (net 7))
 (segment (start 162.56 85.09) (end 167.64 85.09) (width 0.254) (layer "B.Cu") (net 7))
 (segment (start 172.72 85.09) (end 172.72 87.63) (width 0.508) (layer "B.Cu") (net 7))
 (segment (start 175.26 87.63) (end 172.72 87.63) (width 0.508) (layer "B.Cu") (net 7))
 (segment (start 175.26 72.39) (end 172.72 72.39) (width 0.508) (layer "B.Cu") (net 7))
 (segment (start 160.02 90.17) (end 160.02 85.09) (width 0.254) (layer "B.Cu") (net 7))
 (segment (start 124.46 110.49) (end 121.92 110.49) (width 0.508) (layer "B.Cu") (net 7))
 (segment (start 121.92 64.77) (end 121.92 67.31) (width 0.508) (layer "B.Cu") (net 7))
 (segment (start 129.54 105.41) (end 121.92 105.41) (width 0.508) (layer "B.Cu") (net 7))
 (segment (start 124.46 72.39) (end 121.92 72.39) (width 0.508) (layer "B.Cu") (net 7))
 (segment (start 172.72 64.77) (end 172.72 67.31) (width 0.508) (layer "B.Cu") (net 7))
 (segment (start 132.08 64.77) (end 121.92 64.77) (width 0.508) (layer "B.Cu") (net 7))
 (segment (start 170.18 82.55) (end 182.88 82.55) (width 0.254) (layer "F.Cu") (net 1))
 (via (at 170.18 82.55) (size 0.889) (drill 0.635) (layers "F.Cu" "B.Cu") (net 1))
 (via (at 182.88 82.55) (size 0.889) (drill 0.635) (layers "F.Cu" "B.Cu") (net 1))
 (segment (start 119.38 67.31) (end 119.38 72.39) (width 0.508) (layer "B.Cu") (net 1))
 (segment (start 119.38 82.55) (end 119.38 87.63) (width 0.508) (layer "B.Cu") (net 1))
 (segment (start 119.38 123.19) (end 127 123.19) (width 0.508) (layer "B.Cu") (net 1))
 (segment (start 127 123.19) (end 129.54 123.19) (width 0.508) (layer "B.Cu") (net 1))
 (segment (start 119.38 110.49) (end 119.38 123.19) (width 0.508) (layer "B.Cu") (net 1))
 (segment (start 119.38 72.39) (end 119.38 82.55) (width 0.508) (layer "B.Cu") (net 1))
 (segment (start 119.38 100.33) (end 119.38 110.49) (width 0.508) (layer "B.Cu") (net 1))
 (segment (start 119.38 87.63) (end 119.38 100.33) (width 0.508) (layer "B.Cu") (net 1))
 (segment (start 170.18 67.31) (end 170.18 72.39) (width 0.508) (layer "B.Cu") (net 1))
 (segment (start 170.18 123.19) (end 167.64 123.19) (width 0.508) (layer "B.Cu") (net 1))
 (segment (start 170.18 102.87) (end 170.18 123.19) (width 0.508) (layer "B.Cu") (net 1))
 (segment (start 170.18 72.39) (end 170.18 82.55) (width 0.508) (layer "B.Cu") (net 1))
 (segment (start 162.56 64.77) (end 170.18 64.77) (width 0.508) (layer "B.Cu") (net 1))
 (segment (start 182.88 77.47) (end 182.88 82.55) (width 0.254) (layer "B.Cu") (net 1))
 (segment (start 170.18 82.55) (end 170.18 102.87) (width 0.508) (layer "B.Cu") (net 1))
 (segment (start 182.88 82.55) (end 182.88 87.63) (width 0.254) (layer "B.Cu") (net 1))
 (segment (start 119.38 64.77) (end 119.38 67.31) (width 0.508) (layer "B.Cu") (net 1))
 (segment (start 116.84 87.63) (end 119.38 87.63) (width 0.508) (layer "B.Cu") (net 1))
 (segment (start 116.84 92.71) (end 116.84 100.33) (width 0.508) (layer "B.Cu") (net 1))
 (segment (start 167.64 72.39) (end 170.18 72.39) (width 0.508) (layer "B.Cu") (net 1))
 (segment (start 167.64 102.87) (end 170.18 102.87) (width 0.508) (layer "B.Cu") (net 1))
 (segment (start 162.56 67.31) (end 162.56 64.77) (width 0.508) (layer "B.Cu") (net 1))
 (segment (start 170.18 64.77) (end 170.18 67.31) (width 0.508) (layer "B.Cu") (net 1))
 (segment (start 119.38 67.31) (end 111.76 67.31) (width 0.508) (layer "B.Cu") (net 1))
 (segment (start 180.34 77.47) (end 182.88 77.47) (width 0.254) (layer "B.Cu") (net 1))
 (segment (start 116.84 110.49) (end 119.38 110.49) (width 0.508) (layer "B.Cu") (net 1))
 (segment (start 116.84 100.33) (end 119.38 100.33) (width 0.508) (layer "B.Cu") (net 1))
 (segment (start 116.84 72.39) (end 119.38 72.39) (width 0.508) (layer "B.Cu") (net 1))
 (segment (start 175.26 77.47) (end 180.34 77.47) (width 0.254) (layer "B.Cu") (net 1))
 (segment (start 129.54 115.57) (end 124.46 115.57) (width 0.254) (layer "B.Cu") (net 8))
 (segment (start 124.46 115.57) (end 124.46 113.03) (width 0.254) (layer "B.Cu") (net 8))
 (segment (start 129.54 118.11) (end 129.54 115.57) (width 0.254) (layer "B.Cu") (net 8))
 (segment (start 160.02 115.57) (end 160.02 113.03) (width 0.254) (layer "F.Cu") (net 16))
 (segment (start 167.64 115.57) (end 160.02 115.57) (width 0.254) (layer "F.Cu") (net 16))
 (segment (start 162.56 118.11) (end 162.56 100.33) (width 0.254) (layer "B.Cu") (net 23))
 (segment (start 162.56 100.33) (end 167.64 100.33) (width 0.254) (layer "B.Cu") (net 23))
 (segment (start 167.64 118.11) (end 162.56 118.11) (width 0.254) (layer "B.Cu") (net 23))
 (segment (start 175.26 100.33) (end 182.88 100.33) (width 0.254) (layer "B.Cu") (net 18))
 (segment (start 160.02 80.01) (end 167.64 80.01) (width 0.254) (layer "B.Cu") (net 13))
 (segment (start 160.02 67.31) (end 160.02 80.01) (width 0.254) (layer "B.Cu") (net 13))
 (segment (start 167.64 110.49) (end 160.02 110.49) (width 0.254) (layer "F.Cu") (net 15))
 (segment (start 182.88 92.71) (end 182.88 90.17) (width 0.254) (layer "B.Cu") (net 19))
 (segment (start 175.26 92.71) (end 182.88 92.71) (width 0.254) (layer "B.Cu") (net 19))
 (segment (start 182.88 97.79) (end 175.26 97.79) (width 0.254) (layer "B.Cu") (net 17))
 (segment (start 180.34 95.25) (end 180.34 115.57) (width 0.254) (layer "F.Cu") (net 26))
 (segment (start 180.34 115.57) (end 175.26 115.57) (width 0.254) (layer "F.Cu") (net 26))
 (segment (start 180.34 90.17) (end 180.34 95.25) (width 0.254) (layer "F.Cu") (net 26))
 (segment (start 175.26 90.17) (end 180.34 90.17) (width 0.254) (layer "F.Cu") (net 26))
 (segment (start 175.26 95.25) (end 180.34 95.25) (width 0.254) (layer "F.Cu") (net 26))
 (segment (start 111.76 100.33) (end 111.76 107.95) (width 0.254) (layer "B.Cu") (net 2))
 (segment (start 111.76 107.95) (end 111.76 113.03) (width 0.254) (layer "B.Cu") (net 2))
 (segment (start 111.76 113.03) (end 116.84 113.03) (width 0.254) (layer "B.Cu") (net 2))
 (segment (start 111.76 92.71) (end 111.76 100.33) (width 0.254) (layer "B.Cu") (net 2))
 (segment (start 165.1 74.93) (end 167.64 74.93) (width 0.254) (layer "B.Cu") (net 14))
 (segment (start 165.1 67.31) (end 165.1 74.93) (width 0.254) (layer "B.Cu") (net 14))
 (segment (start 162.56 74.93) (end 165.1 74.93) (width 0.254) (layer "B.Cu") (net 14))
 (segment (start 177.8 102.87) (end 177.8 110.49) (width 0.254) (layer "B.Cu") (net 27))
 (segment (start 177.8 110.49) (end 175.26 110.49) (width 0.254) (layer "B.Cu") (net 27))
 (segment (start 175.26 102.87) (end 177.8 102.87) (width 0.254) (layer "B.Cu") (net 27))
 (segment (start 177.8 123.19) (end 177.8 113.03) (width 0.254) (layer "B.Cu") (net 25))
 (segment (start 177.8 113.03) (end 175.26 113.03) (width 0.254) (layer "B.Cu") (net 25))
 (segment (start 175.26 123.19) (end 177.8 123.19) (width 0.254) (layer "B.Cu") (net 25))
 (segment (start 172.72 118.11) (end 172.72 113.03) (width 0.254) (layer "F.Cu") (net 22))
 (segment (start 172.72 113.03) (end 167.64 113.03) (width 0.254) (layer "F.Cu") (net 22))
 (segment (start 175.26 118.11) (end 172.72 118.11) (width 0.254) (layer "F.Cu") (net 22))
 (segment (start 167.64 120.65) (end 175.26 120.65) (width 0.254) (layer "F.Cu") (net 24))
 (segment (start 165.1 77.47) (end 165.1 97.79) (width 0.254) (layer "F.Cu") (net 20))
 (segment (start 165.1 97.79) (end 167.64 97.79) (width 0.254) (layer "F.Cu") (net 20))
 (segment (start 165.1 107.95) (end 167.64 107.95) (width 0.254) (layer "F.Cu") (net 20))
 (segment (start 167.64 77.47) (end 165.1 77.47) (width 0.254) (layer "F.Cu") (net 20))
 (segment (start 165.1 97.79) (end 165.1 107.95) (width 0.254) (layer "F.Cu") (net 20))
 (segment (start 132.08 74.93) (end 124.46 74.93) (width 0.254) (layer "B.Cu") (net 3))
 (segment (start 132.08 91.44) (end 132.08 74.93) (width 0.254) (layer "B.Cu") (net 3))
 (segment (start 129.54 69.85) (end 129.54 77.47) (width 0.254) (layer "F.Cu") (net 10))
 (segment (start 111.76 69.85) (end 129.54 69.85) (width 0.254) (layer "F.Cu") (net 10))
 (segment (start 111.76 74.93) (end 111.76 69.85) (width 0.254) (layer "B.Cu") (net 10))
 (segment (start 129.54 77.47) (end 124.46 77.47) (width 0.254) (layer "B.Cu") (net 10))
 (segment (start 116.84 74.93) (end 111.76 74.93) (width 0.254) (layer "B.Cu") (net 10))
 (segment (start 175.26 80.01) (end 180.34 80.01) (width 0.254) (layer "B.Cu") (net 21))
 (segment (start 111.76 87.63) (end 114.3 87.63) (width 0.254) (layer "B.Cu") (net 6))
 (segment (start 109.22 77.47) (end 109.22 110.49) (width 0.254) (layer "B.Cu") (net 5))
 (segment (start 116.84 77.47) (end 111.76 77.47) (width 0.254) (layer "B.Cu") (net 5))
 (segment (start 111.76 77.47) (end 109.22 77.47) (width 0.254) (layer "B.Cu") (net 5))
 (segment (start 124.46 80.01) (end 124.46 82.55) (width 0.254) (layer "B.Cu") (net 11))
 (segment (start 129.54 101.6) (end 129.54 87.63) (width 0.254) (layer "B.Cu") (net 4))
 (segment (start 109.22 115.57) (end 116.84 115.57) (width 0.254) (layer "B.Cu") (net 9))
 (segment (start 109.22 113.03) (end 109.22 115.57) (width 0.254) (layer "B.Cu") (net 9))
 (segment (start 124.46 118.11) (end 127 118.11) (width 0.254) (layer "B.Cu") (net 12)))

